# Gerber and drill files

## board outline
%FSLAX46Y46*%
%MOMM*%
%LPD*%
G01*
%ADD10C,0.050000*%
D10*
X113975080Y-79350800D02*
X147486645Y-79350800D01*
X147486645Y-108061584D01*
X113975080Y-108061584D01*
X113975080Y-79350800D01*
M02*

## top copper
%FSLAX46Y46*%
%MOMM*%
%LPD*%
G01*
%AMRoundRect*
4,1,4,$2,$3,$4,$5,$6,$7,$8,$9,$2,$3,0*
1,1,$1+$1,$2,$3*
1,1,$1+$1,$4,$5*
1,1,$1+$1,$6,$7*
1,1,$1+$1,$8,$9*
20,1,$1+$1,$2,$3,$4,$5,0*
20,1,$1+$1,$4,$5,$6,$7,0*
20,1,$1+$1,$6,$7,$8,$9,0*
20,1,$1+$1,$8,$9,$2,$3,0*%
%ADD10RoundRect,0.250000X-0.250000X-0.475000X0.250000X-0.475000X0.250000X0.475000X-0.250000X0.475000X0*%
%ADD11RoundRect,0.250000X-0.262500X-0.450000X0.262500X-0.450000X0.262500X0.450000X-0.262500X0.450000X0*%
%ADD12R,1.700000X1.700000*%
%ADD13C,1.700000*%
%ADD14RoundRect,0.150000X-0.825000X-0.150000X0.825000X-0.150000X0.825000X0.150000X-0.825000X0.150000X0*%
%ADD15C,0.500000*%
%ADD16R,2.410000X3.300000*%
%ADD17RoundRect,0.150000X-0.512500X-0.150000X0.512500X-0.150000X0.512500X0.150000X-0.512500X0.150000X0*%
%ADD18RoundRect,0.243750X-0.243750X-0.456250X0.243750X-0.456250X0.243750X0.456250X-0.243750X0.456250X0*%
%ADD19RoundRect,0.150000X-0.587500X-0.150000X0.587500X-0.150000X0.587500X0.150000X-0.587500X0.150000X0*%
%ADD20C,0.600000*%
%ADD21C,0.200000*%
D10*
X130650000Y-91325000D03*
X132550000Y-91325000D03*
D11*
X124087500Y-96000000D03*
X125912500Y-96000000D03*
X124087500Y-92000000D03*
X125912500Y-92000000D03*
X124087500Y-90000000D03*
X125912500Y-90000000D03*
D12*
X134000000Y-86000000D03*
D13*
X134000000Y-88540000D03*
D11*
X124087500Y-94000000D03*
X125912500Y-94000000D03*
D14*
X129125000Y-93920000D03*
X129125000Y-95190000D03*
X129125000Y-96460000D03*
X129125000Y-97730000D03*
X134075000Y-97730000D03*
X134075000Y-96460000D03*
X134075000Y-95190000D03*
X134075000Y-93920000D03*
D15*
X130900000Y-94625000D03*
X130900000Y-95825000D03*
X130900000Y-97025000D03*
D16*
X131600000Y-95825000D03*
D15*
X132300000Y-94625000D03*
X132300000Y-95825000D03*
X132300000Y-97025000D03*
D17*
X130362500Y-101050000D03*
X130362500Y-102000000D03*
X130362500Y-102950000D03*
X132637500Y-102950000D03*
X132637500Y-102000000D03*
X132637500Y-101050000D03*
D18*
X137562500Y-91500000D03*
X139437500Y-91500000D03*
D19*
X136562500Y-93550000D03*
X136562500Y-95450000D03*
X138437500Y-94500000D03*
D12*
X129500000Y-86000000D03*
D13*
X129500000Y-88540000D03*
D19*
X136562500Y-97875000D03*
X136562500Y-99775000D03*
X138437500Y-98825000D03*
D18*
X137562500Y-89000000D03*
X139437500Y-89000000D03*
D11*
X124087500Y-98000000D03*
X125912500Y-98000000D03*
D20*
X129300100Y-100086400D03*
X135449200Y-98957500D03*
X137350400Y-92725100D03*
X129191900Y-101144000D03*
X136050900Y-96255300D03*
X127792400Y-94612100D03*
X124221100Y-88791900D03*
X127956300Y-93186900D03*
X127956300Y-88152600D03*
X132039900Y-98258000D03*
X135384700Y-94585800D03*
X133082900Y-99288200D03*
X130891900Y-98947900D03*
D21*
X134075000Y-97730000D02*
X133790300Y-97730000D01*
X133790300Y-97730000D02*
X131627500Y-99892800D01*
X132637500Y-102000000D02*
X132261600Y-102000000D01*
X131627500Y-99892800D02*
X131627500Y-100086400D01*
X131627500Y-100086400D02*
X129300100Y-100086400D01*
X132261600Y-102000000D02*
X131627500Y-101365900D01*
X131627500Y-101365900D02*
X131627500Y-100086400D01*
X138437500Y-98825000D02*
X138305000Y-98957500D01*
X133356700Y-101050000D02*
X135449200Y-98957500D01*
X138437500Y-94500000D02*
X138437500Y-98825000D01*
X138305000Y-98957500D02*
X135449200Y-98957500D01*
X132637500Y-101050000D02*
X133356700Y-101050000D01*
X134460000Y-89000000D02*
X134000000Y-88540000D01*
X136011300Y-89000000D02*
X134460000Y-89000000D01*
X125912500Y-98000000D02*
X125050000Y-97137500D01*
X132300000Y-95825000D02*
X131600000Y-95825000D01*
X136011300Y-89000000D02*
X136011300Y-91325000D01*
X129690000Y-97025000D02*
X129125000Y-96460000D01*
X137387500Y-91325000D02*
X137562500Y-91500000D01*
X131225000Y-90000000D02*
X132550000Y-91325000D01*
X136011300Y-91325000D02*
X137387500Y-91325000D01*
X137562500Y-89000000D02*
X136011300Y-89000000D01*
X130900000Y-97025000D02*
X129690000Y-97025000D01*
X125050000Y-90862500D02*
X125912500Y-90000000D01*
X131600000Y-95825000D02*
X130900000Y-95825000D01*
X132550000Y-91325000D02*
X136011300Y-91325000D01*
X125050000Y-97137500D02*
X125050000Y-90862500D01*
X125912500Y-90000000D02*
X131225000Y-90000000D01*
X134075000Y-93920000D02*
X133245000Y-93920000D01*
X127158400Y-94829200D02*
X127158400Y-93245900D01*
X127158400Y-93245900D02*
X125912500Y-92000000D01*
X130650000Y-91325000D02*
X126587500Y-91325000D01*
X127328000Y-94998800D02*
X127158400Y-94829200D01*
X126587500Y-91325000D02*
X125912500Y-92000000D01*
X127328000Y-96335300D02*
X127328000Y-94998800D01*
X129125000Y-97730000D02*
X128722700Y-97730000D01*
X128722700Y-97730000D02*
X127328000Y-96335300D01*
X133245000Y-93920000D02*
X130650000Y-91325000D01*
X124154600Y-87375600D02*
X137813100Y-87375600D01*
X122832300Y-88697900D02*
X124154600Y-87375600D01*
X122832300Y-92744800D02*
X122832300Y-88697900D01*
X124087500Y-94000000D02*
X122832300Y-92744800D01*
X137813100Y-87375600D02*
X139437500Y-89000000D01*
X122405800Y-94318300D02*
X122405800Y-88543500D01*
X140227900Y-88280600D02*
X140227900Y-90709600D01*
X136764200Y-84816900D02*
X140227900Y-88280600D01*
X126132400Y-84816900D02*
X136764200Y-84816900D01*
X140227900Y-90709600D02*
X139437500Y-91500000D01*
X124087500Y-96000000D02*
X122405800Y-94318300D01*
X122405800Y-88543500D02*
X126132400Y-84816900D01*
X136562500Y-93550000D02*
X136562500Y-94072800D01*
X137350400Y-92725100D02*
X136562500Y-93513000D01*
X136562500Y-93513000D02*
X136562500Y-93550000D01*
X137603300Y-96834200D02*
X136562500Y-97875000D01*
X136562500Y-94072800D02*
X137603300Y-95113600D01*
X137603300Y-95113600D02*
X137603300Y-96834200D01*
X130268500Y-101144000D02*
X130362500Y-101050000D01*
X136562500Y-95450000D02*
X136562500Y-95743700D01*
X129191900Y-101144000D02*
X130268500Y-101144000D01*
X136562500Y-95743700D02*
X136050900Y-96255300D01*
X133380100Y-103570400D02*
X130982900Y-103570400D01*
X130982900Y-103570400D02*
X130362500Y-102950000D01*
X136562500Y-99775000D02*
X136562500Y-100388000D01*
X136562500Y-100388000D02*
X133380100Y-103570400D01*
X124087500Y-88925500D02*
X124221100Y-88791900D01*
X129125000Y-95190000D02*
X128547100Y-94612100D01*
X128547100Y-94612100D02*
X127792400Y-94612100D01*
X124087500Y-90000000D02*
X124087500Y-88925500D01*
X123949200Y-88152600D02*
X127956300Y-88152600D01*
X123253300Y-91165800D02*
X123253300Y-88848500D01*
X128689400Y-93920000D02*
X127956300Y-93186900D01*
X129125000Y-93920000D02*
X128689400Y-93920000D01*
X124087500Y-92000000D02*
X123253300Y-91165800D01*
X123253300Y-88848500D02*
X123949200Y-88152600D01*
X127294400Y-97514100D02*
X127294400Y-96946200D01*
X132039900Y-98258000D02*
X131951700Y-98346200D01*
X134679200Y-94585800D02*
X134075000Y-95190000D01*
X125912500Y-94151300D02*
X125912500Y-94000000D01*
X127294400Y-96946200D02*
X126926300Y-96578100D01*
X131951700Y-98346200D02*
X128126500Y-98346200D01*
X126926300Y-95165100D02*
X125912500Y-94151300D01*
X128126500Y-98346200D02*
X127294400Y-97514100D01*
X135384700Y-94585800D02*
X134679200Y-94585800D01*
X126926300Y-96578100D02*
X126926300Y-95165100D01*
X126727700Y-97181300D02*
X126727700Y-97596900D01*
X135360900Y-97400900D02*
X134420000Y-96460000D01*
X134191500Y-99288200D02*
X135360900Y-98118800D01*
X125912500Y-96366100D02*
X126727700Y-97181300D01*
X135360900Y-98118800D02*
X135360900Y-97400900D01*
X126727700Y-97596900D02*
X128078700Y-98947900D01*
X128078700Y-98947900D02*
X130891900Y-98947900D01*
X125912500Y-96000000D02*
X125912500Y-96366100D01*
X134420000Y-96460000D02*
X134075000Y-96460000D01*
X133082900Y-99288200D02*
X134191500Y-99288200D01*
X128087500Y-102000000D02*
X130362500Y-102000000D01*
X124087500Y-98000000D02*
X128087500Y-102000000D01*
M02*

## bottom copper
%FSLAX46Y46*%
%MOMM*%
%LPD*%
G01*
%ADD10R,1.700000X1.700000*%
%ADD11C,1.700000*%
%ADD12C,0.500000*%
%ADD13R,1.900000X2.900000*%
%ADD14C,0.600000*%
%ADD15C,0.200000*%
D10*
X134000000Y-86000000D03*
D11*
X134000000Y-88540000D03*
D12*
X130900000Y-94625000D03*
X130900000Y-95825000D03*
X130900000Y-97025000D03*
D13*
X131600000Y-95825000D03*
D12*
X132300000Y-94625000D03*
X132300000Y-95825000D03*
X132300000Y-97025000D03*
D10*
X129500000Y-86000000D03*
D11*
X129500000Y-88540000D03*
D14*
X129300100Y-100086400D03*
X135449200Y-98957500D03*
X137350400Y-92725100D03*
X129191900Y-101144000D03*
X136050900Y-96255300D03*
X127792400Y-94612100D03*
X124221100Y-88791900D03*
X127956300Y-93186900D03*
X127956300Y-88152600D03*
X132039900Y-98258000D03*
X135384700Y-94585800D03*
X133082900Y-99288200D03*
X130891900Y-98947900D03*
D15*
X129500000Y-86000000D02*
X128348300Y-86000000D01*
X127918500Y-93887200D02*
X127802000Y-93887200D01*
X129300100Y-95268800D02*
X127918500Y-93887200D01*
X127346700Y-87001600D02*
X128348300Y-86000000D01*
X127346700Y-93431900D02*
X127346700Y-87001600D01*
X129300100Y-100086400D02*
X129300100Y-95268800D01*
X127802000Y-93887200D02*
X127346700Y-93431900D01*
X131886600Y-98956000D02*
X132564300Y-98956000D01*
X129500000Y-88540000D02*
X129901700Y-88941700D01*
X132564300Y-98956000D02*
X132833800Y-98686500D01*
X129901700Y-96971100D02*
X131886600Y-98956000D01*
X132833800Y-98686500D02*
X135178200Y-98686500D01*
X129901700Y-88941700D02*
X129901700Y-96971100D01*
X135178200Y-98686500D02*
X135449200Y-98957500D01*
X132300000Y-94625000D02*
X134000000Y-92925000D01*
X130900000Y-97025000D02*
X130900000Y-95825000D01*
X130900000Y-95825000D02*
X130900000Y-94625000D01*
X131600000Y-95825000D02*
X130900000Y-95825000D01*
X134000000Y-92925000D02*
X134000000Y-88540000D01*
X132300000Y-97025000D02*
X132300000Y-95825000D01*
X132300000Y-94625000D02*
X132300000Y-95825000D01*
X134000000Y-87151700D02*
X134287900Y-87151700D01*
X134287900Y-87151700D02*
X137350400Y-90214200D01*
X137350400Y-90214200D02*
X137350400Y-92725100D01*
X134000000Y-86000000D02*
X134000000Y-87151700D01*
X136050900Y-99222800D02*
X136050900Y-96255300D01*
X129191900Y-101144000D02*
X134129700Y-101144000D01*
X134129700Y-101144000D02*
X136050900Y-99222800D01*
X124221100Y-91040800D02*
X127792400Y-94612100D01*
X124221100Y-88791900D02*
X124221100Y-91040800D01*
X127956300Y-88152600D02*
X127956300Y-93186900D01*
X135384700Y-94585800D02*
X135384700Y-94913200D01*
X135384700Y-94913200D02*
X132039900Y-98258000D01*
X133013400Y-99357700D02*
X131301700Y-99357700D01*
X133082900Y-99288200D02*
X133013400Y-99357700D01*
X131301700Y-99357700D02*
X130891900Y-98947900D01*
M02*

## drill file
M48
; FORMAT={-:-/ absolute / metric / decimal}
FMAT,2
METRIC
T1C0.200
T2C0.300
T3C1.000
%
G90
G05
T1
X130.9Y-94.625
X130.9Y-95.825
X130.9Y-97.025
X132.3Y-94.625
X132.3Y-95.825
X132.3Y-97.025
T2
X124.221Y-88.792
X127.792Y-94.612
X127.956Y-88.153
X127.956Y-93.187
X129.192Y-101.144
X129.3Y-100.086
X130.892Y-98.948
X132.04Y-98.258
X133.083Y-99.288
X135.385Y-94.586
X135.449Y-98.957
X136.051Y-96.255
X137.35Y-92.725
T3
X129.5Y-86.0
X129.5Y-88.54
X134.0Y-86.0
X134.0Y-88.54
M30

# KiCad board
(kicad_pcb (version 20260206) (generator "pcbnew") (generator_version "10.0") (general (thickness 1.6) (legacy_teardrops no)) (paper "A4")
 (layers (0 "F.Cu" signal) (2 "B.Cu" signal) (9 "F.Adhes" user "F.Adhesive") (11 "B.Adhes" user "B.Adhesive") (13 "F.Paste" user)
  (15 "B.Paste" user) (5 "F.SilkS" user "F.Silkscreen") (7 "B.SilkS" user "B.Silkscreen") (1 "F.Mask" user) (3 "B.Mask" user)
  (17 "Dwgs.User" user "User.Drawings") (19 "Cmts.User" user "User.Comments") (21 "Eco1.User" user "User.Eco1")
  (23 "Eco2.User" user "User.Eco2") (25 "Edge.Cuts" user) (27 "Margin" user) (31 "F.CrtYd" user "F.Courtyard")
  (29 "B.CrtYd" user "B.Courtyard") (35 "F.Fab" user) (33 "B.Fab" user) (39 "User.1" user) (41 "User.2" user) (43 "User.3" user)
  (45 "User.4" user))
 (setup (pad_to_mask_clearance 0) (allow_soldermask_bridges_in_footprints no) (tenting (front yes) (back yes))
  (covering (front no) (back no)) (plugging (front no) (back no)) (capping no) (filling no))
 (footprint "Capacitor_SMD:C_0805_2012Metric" (layer "F.Cu") (at 131.6 91.325)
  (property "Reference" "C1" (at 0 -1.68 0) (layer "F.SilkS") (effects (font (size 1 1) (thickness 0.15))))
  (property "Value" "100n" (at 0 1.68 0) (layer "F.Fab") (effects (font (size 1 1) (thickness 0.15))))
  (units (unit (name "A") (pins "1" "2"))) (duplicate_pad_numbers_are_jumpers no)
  (pad "1" smd roundrect (at -0.95 0) (size 1 1.45) (layers "F.Cu" "F.Mask" "F.Paste") (roundrect_rratio 0.25) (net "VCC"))
  (pad "2" smd roundrect (at 0.95 0) (size 1 1.45) (layers "F.Cu" "F.Mask" "F.Paste") (roundrect_rratio 0.25) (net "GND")))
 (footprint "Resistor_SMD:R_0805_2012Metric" (layer "F.Cu") (at 125 96)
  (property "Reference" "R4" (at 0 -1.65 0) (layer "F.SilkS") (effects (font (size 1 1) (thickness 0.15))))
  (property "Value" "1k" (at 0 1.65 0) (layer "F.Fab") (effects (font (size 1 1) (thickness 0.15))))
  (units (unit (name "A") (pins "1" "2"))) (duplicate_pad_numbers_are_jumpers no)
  (pad "1" smd roundrect (at -0.9125 0) (size 1.025 1.4) (layers "F.Cu" "F.Mask" "F.Paste") (roundrect_rratio 0.243902) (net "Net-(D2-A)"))
  (pad "2" smd roundrect (at 0.9125 0) (size 1.025 1.4) (layers "F.Cu" "F.Mask" "F.Paste") (roundrect_rratio 0.243902)
   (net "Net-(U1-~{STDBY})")))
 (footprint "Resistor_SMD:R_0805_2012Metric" (layer "F.Cu") (at 125 92)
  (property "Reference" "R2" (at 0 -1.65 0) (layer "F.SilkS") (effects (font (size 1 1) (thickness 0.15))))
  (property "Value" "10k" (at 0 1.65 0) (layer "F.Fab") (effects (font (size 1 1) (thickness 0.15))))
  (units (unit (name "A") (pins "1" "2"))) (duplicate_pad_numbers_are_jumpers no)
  (pad "1" smd roundrect (at -0.9125 0) (size 1.025 1.4) (layers "F.Cu" "F.Mask" "F.Paste") (roundrect_rratio 0.243902)
   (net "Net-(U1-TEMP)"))
  (pad "2" smd roundrect (at 0.9125 0) (size 1.025 1.4) (layers "F.Cu" "F.Mask" "F.Paste") (roundrect_rratio 0.243902) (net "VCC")))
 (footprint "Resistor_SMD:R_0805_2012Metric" (layer "F.Cu") (at 125 90)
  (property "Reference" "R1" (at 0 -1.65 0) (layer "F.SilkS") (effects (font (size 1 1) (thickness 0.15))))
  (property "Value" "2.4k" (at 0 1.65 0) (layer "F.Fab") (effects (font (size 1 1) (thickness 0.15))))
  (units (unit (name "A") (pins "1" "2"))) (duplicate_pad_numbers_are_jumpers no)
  (pad "1" smd roundrect (at -0.9125 0) (size 1.025 1.4) (layers "F.Cu" "F.Mask" "F.Paste") (roundrect_rratio 0.243902)
   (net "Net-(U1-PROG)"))
  (pad "2" smd roundrect (at 0.9125 0) (size 1.025 1.4) (layers "F.Cu" "F.Mask" "F.Paste") (roundrect_rratio 0.243902) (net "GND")))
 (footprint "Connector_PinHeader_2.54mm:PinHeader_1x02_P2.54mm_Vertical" (layer "F.Cu") (at 134 86)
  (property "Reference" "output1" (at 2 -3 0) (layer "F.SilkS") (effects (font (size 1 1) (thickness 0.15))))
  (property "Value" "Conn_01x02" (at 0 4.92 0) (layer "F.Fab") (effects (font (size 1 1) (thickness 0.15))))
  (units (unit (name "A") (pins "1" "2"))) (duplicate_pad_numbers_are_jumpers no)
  (pad "1" thru_hole rect (at 0 0) (size 1.7 1.7) (drill 1) (layers "*.Cu" "*.Mask") (remove_unused_layers no) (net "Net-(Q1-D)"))
  (pad "2" thru_hole circle (at 0 2.54) (size 1.7 1.7) (drill 1) (layers "*.Cu" "*.Mask") (remove_unused_layers no) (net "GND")))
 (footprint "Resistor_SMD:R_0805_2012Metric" (layer "F.Cu") (at 125 94)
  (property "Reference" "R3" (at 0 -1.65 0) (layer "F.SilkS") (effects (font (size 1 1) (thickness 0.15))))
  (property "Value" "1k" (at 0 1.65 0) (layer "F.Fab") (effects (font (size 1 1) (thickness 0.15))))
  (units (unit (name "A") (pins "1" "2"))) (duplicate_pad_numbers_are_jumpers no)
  (pad "1" smd roundrect (at -0.9125 0) (size 1.025 1.4) (layers "F.Cu" "F.Mask" "F.Paste") (roundrect_rratio 0.243902) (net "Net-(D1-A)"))
  (pad "2" smd roundrect (at 0.9125 0) (size 1.025 1.4) (layers "F.Cu" "F.Mask" "F.Paste") (roundrect_rratio 0.243902)
   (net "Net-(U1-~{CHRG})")))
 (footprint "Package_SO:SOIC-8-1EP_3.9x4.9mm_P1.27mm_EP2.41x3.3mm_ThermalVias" (layer "F.Cu") (at 131.6 95.825)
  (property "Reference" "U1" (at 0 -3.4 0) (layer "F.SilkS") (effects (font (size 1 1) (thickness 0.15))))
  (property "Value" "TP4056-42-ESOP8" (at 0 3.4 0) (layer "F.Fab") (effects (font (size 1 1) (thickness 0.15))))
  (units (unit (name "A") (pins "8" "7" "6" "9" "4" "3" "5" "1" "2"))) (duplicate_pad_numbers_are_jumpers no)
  (pad "" smd roundrect (at -0.6 -0.825) (size 1.01 1.38) (layers "F.Paste") (roundrect_rratio 0.247525))
  (pad "" smd roundrect (at -0.6 0.825) (size 1.01 1.38) (layers "F.Paste") (roundrect_rratio 0.247525))
  (pad "" smd roundrect (at 0.6 -0.825) (size 1.01 1.38) (layers "F.Paste") (roundrect_rratio 0.247525))
  (pad "" smd roundrect (at 0.6 0.825) (size 1.01 1.38) (layers "F.Paste") (roundrect_rratio 0.247525))
  (pad "1" smd roundrect (at -2.475 -1.905) (size 1.95 0.6) (layers "F.Cu" "F.Mask" "F.Paste") (roundrect_rratio 0.25) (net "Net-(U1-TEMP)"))
  (pad "2" smd roundrect (at -2.475 -0.635) (size 1.95 0.6) (layers "F.Cu" "F.Mask" "F.Paste") (roundrect_rratio 0.25) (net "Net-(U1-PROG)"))
  (pad "3" smd roundrect (at -2.475 0.635) (size 1.95 0.6) (layers "F.Cu" "F.Mask" "F.Paste") (roundrect_rratio 0.25) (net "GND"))
  (pad "4" smd roundrect (at -2.475 1.905) (size 1.95 0.6) (layers "F.Cu" "F.Mask" "F.Paste") (roundrect_rratio 0.25) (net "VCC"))
  (pad "5" smd roundrect (at 2.475 1.905) (size 1.95 0.6) (layers "F.Cu" "F.Mask" "F.Paste") (roundrect_rratio 0.25) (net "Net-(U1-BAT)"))
  (pad "6" smd roundrect (at 2.475 0.635) (size 1.95 0.6) (layers "F.Cu" "F.Mask" "F.Paste") (roundrect_rratio 0.25)
   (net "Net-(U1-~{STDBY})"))
  (pad "7" smd roundrect (at 2.475 -0.635) (size 1.95 0.6) (layers "F.Cu" "F.Mask" "F.Paste") (roundrect_rratio 0.25)
   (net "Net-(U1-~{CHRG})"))
  (pad "8" smd roundrect (at 2.475 -1.905) (size 1.95 0.6) (layers "F.Cu" "F.Mask" "F.Paste") (roundrect_rratio 0.25) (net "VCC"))
  (pad "9" thru_hole circle (at -0.7 -1.2) (size 0.5 0.5) (drill 0.2) (layers "*.Cu") (remove_unused_layers no) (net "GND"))
  (pad "9" thru_hole circle (at -0.7 0) (size 0.5 0.5) (drill 0.2) (layers "*.Cu") (remove_unused_layers no) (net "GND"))
  (pad "9" thru_hole circle (at -0.7 1.2) (size 0.5 0.5) (drill 0.2) (layers "*.Cu") (remove_unused_layers no) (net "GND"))
  (pad "9" smd rect (at 0 0) (size 1.9 2.9) (layers "B.Cu") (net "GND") (zone_connect 2))
  (pad "9" smd rect (at 0 0) (size 2.41 3.3) (layers "F.Cu" "F.Mask") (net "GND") (zone_connect 2))
  (pad "9" thru_hole circle (at 0.7 -1.2) (size 0.5 0.5) (drill 0.2) (layers "*.Cu") (remove_unused_layers no) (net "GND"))
  (pad "9" thru_hole circle (at 0.7 0) (size 0.5 0.5) (drill 0.2) (layers "*.Cu") (remove_unused_layers no) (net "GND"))
  (pad "9" thru_hole circle (at 0.7 1.2) (size 0.5 0.5) (drill 0.2) (layers "*.Cu") (remove_unused_layers no) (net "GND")))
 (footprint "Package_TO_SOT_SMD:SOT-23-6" (layer "F.Cu") (at 131.5 102)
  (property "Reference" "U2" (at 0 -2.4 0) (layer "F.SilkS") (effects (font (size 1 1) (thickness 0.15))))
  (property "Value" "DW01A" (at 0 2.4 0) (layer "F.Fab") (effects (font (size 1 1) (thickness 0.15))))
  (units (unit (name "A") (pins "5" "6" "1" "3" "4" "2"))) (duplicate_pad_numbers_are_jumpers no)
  (pad "1" smd roundrect (at -1.1375 -0.95) (size 1.325 0.6) (layers "F.Cu" "F.Mask" "F.Paste") (roundrect_rratio 0.25) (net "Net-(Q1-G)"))
  (pad "2" smd roundrect (at -1.1375 0) (size 1.325 0.6) (layers "F.Cu" "F.Mask" "F.Paste") (roundrect_rratio 0.25) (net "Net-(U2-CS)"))
  (pad "3" smd roundrect (at -1.1375 0.95) (size 1.325 0.6) (layers "F.Cu" "F.Mask" "F.Paste") (roundrect_rratio 0.25) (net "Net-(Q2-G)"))
  (pad "4" smd roundrect (at 1.1375 0.95) (size 1.325 0.6) (layers "F.Cu" "F.Mask" "F.Paste") (roundrect_rratio 0.25)
   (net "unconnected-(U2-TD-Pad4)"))
  (pad "5" smd roundrect (at 1.1375 0) (size 1.325 0.6) (layers "F.Cu" "F.Mask" "F.Paste") (roundrect_rratio 0.25) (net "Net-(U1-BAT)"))
  (pad "6" smd roundrect (at 1.1375 -0.95) (size 1.325 0.6) (layers "F.Cu" "F.Mask" "F.Paste") (roundrect_rratio 0.25) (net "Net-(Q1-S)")))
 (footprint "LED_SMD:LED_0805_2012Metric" (layer "F.Cu") (at 138.5 91.5)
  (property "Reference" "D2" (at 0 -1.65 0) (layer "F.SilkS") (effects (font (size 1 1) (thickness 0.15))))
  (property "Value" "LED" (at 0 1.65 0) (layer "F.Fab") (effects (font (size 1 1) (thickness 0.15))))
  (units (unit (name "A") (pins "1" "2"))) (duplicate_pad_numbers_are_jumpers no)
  (pad "1" smd roundrect (at -0.9375 0) (size 0.975 1.4) (layers "F.Cu" "F.Mask" "F.Paste") (roundrect_rratio 0.25) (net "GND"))
  (pad "2" smd roundrect (at 0.9375 0) (size 0.975 1.4) (layers "F.Cu" "F.Mask" "F.Paste") (roundrect_rratio 0.25) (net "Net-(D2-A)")))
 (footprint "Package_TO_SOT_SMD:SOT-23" (layer "F.Cu") (at 137.5 94.5)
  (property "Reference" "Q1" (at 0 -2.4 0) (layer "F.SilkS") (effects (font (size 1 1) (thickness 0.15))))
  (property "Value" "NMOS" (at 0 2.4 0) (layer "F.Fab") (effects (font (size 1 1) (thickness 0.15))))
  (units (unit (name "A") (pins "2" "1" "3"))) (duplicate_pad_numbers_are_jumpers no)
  (pad "1" smd roundrect (at -0.9375 -0.95) (size 1.475 0.6) (layers "F.Cu" "F.Mask" "F.Paste") (roundrect_rratio 0.25) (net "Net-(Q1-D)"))
  (pad "2" smd roundrect (at -0.9375 0.95) (size 1.475 0.6) (layers "F.Cu" "F.Mask" "F.Paste") (roundrect_rratio 0.25) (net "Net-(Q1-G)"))
  (pad "3" smd roundrect (at 0.9375 0) (size 1.475 0.6) (layers "F.Cu" "F.Mask" "F.Paste") (roundrect_rratio 0.25) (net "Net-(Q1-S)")))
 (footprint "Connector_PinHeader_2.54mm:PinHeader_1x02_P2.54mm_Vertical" (layer "F.Cu") (at 129.5 86)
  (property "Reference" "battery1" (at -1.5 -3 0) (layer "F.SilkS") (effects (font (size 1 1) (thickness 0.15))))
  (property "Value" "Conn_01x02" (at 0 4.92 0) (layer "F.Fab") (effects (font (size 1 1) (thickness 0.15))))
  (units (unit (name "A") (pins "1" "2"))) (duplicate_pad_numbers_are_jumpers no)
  (pad "1" thru_hole rect (at 0 0) (size 1.7 1.7) (drill 1) (layers "*.Cu" "*.Mask") (remove_unused_layers no) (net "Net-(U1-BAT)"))
  (pad "2" thru_hole circle (at 0 2.54) (size 1.7 1.7) (drill 1) (layers "*.Cu" "*.Mask") (remove_unused_layers no) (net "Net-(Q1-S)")))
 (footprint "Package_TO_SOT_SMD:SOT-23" (layer "F.Cu") (at 137.5 98.825)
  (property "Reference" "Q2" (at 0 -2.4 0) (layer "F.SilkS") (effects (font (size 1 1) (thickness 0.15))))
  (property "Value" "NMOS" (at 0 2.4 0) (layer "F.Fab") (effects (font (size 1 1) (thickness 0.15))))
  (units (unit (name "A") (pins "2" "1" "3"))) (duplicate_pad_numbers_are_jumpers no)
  (pad "1" smd roundrect (at -0.9375 -0.95) (size 1.475 0.6) (layers "F.Cu" "F.Mask" "F.Paste") (roundrect_rratio 0.25) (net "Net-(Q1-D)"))
  (pad "2" smd roundrect (at -0.9375 0.95) (size 1.475 0.6) (layers "F.Cu" "F.Mask" "F.Paste") (roundrect_rratio 0.25) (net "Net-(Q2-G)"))
  (pad "3" smd roundrect (at 0.9375 0) (size 1.475 0.6) (layers "F.Cu" "F.Mask" "F.Paste") (roundrect_rratio 0.25) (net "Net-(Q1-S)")))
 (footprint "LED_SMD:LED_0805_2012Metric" (layer "F.Cu") (at 138.5 89)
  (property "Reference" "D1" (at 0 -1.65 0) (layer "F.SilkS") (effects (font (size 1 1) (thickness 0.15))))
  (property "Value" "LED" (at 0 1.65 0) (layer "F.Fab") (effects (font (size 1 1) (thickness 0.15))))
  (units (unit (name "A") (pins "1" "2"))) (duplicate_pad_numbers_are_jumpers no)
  (pad "1" smd roundrect (at -0.9375 0) (size 0.975 1.4) (layers "F.Cu" "F.Mask" "F.Paste") (roundrect_rratio 0.25) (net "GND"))
  (pad "2" smd roundrect (at 0.9375 0) (size 0.975 1.4) (layers "F.Cu" "F.Mask" "F.Paste") (roundrect_rratio 0.25) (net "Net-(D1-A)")))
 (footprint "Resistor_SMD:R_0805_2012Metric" (layer "F.Cu") (at 125 98)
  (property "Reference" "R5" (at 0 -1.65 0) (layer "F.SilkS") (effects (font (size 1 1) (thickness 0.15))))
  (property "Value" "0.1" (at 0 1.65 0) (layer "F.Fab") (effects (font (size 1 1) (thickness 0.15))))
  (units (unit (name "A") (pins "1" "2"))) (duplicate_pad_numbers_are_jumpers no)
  (pad "1" smd roundrect (at -0.9125 0) (size 1.025 1.4) (layers "F.Cu" "F.Mask" "F.Paste") (roundrect_rratio 0.243902) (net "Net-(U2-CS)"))
  (pad "2" smd roundrect (at 0.9125 0) (size 1.025 1.4) (layers "F.Cu" "F.Mask" "F.Paste") (roundrect_rratio 0.243902) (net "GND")))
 (gr_rect (start 113.97508 79.3508) (end 147.486645 108.061584) (stroke (width 0.05) (type default)) (fill no) (layer "Edge.Cuts"))
 (segment (start 134.075 97.73) (end 133.7903 97.73) (width 0.2) (layer "F.Cu") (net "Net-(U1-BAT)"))
 (segment (start 133.7903 97.73) (end 131.6275 99.8928) (width 0.2) (layer "F.Cu") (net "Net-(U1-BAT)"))
 (segment (start 132.6375 102) (end 132.2616 102) (width 0.2) (layer "F.Cu") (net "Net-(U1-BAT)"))
 (segment (start 131.6275 99.8928) (end 131.6275 100.0864) (width 0.2) (layer "F.Cu") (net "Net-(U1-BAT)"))
 (segment (start 131.6275 100.0864) (end 129.3001 100.0864) (width 0.2) (layer "F.Cu") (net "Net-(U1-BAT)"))
 (segment (start 132.2616 102) (end 131.6275 101.3659) (width 0.2) (layer "F.Cu") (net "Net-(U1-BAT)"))
 (segment (start 131.6275 101.3659) (end 131.6275 100.0864) (width 0.2) (layer "F.Cu") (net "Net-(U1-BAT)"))
 (via (at 129.3001 100.0864) (size 0.6) (drill 0.3) (layers "F.Cu" "B.Cu") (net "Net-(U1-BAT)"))
 (segment (start 129.5 86) (end 128.3483 86) (width 0.2) (layer "B.Cu") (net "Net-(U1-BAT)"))
 (segment (start 127.9185 93.8872) (end 127.802 93.8872) (width 0.2) (layer "B.Cu") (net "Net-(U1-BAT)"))
 (segment (start 129.3001 95.2688) (end 127.9185 93.8872) (width 0.2) (layer "B.Cu") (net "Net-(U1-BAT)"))
 (segment (start 127.3467 87.0016) (end 128.3483 86) (width 0.2) (layer "B.Cu") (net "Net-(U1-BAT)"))
 (segment (start 127.3467 93.4319) (end 127.3467 87.0016) (width 0.2) (layer "B.Cu") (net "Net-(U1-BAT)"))
 (segment (start 129.3001 100.0864) (end 129.3001 95.2688) (width 0.2) (layer "B.Cu") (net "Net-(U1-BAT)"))
 (segment (start 127.802 93.8872) (end 127.3467 93.4319) (width 0.2) (layer "B.Cu") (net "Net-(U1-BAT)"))
 (segment (start 138.4375 98.825) (end 138.305 98.9575) (width 0.2) (layer "F.Cu") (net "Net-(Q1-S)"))
 (segment (start 133.3567 101.05) (end 135.4492 98.9575) (width 0.2) (layer "F.Cu") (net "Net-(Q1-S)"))
 (segment (start 138.4375 94.5) (end 138.4375 98.825) (width 0.2) (layer "F.Cu") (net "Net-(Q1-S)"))
 (segment (start 138.305 98.9575) (end 135.4492 98.9575) (width 0.2) (layer "F.Cu") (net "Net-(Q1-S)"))
 (segment (start 132.6375 101.05) (end 133.3567 101.05) (width 0.2) (layer "F.Cu") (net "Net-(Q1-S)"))
 (via (at 135.4492 98.9575) (size 0.6) (drill 0.3) (layers "F.Cu" "B.Cu") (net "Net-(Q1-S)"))
 (segment (start 131.8866 98.956) (end 132.5643 98.956) (width 0.2) (layer "B.Cu") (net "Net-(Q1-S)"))
 (segment (start 129.5 88.54) (end 129.9017 88.9417) (width 0.2) (layer "B.Cu") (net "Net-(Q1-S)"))
 (segment (start 132.5643 98.956) (end 132.8338 98.6865) (width 0.2) (layer "B.Cu") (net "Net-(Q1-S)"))
 (segment (start 129.9017 96.9711) (end 131.8866 98.956) (width 0.2) (layer "B.Cu") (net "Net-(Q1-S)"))
 (segment (start 132.8338 98.6865) (end 135.1782 98.6865) (width 0.2) (layer "B.Cu") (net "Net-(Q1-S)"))
 (segment (start 129.9017 88.9417) (end 129.9017 96.9711) (width 0.2) (layer "B.Cu") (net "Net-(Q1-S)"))
 (segment (start 135.1782 98.6865) (end 135.4492 98.9575) (width 0.2) (layer "B.Cu") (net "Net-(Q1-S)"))
 (segment (start 134.46 89) (end 134 88.54) (width 0.2) (layer "F.Cu") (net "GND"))
 (segment (start 136.0113 89) (end 134.46 89) (width 0.2) (layer "F.Cu") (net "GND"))
 (segment (start 125.9125 98) (end 125.05 97.1375) (width 0.2) (layer "F.Cu") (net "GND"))
 (segment (start 132.3 95.825) (end 131.6 95.825) (width 0.2) (layer "F.Cu") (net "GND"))
 (segment (start 136.0113 89) (end 136.0113 91.325) (width 0.2) (layer "F.Cu") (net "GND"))
 (segment (start 129.69 97.025) (end 129.125 96.46) (width 0.2) (layer "F.Cu") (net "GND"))
 (segment (start 137.3875 91.325) (end 137.5625 91.5) (width 0.2) (layer "F.Cu") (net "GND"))
 (segment (start 131.225 90) (end 132.55 91.325) (width 0.2) (layer "F.Cu") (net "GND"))
 (segment (start 136.0113 91.325) (end 137.3875 91.325) (width 0.2) (layer "F.Cu") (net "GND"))
 (segment (start 137.5625 89) (end 136.0113 89) (width 0.2) (layer "F.Cu") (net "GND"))
 (segment (start 130.9 97.025) (end 129.69 97.025) (width 0.2) (layer "F.Cu") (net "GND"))
 (segment (start 125.05 90.8625) (end 125.9125 90) (width 0.2) (layer "F.Cu") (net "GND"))
 (segment (start 131.6 95.825) (end 130.9 95.825) (width 0.2) (layer "F.Cu") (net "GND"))
 (segment (start 132.55 91.325) (end 136.0113 91.325) (width 0.2) (layer "F.Cu") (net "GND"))
 (segment (start 125.05 97.1375) (end 125.05 90.8625) (width 0.2) (layer "F.Cu") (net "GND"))
 (segment (start 125.9125 90) (end 131.225 90) (width 0.2) (layer "F.Cu") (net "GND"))
 (segment (start 132.3 94.625) (end 134 92.925) (width 0.2) (layer "B.Cu") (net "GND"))
 (segment (start 130.9 97.025) (end 130.9 95.825) (width 0.2) (layer "B.Cu") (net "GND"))
 (segment (start 130.9 95.825) (end 130.9 94.625) (width 0.2) (layer "B.Cu") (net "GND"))
 (segment (start 131.6 95.825) (end 130.9 95.825) (width 0.2) (layer "B.Cu") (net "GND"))
 (segment (start 134 92.925) (end 134 88.54) (width 0.2) (layer "B.Cu") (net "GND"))
 (segment (start 132.3 97.025) (end 132.3 95.825) (width 0.2) (layer "B.Cu") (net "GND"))
 (segment (start 132.3 94.625) (end 132.3 95.825) (width 0.2) (layer "B.Cu") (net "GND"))
 (segment (start 134.075 93.92) (end 133.245 93.92) (width 0.2) (layer "F.Cu") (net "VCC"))
 (segment (start 127.1584 94.8292) (end 127.1584 93.2459) (width 0.2) (layer "F.Cu") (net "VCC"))
 (segment (start 127.1584 93.2459) (end 125.9125 92) (width 0.2) (layer "F.Cu") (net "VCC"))
 (segment (start 130.65 91.325) (end 126.5875 91.325) (width 0.2) (layer "F.Cu") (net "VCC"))
 (segment (start 127.328 94.9988) (end 127.1584 94.8292) (width 0.2) (layer "F.Cu") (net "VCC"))
 (segment (start 126.5875 91.325) (end 125.9125 92) (width 0.2) (layer "F.Cu") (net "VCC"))
 (segment (start 127.328 96.3353) (end 127.328 94.9988) (width 0.2) (layer "F.Cu") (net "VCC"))
 (segment (start 129.125 97.73) (end 128.7227 97.73) (width 0.2) (layer "F.Cu") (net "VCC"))
 (segment (start 128.7227 97.73) (end 127.328 96.3353) (width 0.2) (layer "F.Cu") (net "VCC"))
 (segment (start 133.245 93.92) (end 130.65 91.325) (width 0.2) (layer "F.Cu") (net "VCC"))
 (segment (start 124.1546 87.3756) (end 137.8131 87.3756) (width 0.2) (layer "F.Cu") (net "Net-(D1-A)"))
 (segment (start 122.8323 88.6979) (end 124.1546 87.3756) (width 0.2) (layer "F.Cu") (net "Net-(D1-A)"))
 (segment (start 122.8323 92.7448) (end 122.8323 88.6979) (width 0.2) (layer "F.Cu") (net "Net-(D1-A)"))
 (segment (start 124.0875 94) (end 122.8323 92.7448) (width 0.2) (layer "F.Cu") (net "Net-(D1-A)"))
 (segment (start 137.8131 87.3756) (end 139.4375 89) (width 0.2) (layer "F.Cu") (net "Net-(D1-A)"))
 (segment (start 122.4058 94.3183) (end 122.4058 88.5435) (width 0.2) (layer "F.Cu") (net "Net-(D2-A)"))
 (segment (start 140.2279 88.2806) (end 140.2279 90.7096) (width 0.2) (layer "F.Cu") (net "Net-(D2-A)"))
 (segment (start 136.7642 84.8169) (end 140.2279 88.2806) (width 0.2) (layer "F.Cu") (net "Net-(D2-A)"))
 (segment (start 126.1324 84.8169) (end 136.7642 84.8169) (width 0.2) (layer "F.Cu") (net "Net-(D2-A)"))
 (segment (start 140.2279 90.7096) (end 139.4375 91.5) (width 0.2) (layer "F.Cu") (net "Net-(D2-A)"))
 (segment (start 124.0875 96) (end 122.4058 94.3183) (width 0.2) (layer "F.Cu") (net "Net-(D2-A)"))
 (segment (start 122.4058 88.5435) (end 126.1324 84.8169) (width 0.2) (layer "F.Cu") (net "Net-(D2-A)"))
 (segment (start 136.5625 93.55) (end 136.5625 94.0728) (width 0.2) (layer "F.Cu") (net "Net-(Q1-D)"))
 (segment (start 137.3504 92.7251) (end 136.5625 93.513) (width 0.2) (layer "F.Cu") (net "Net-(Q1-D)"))
 (segment (start 136.5625 93.513) (end 136.5625 93.55) (width 0.2) (layer "F.Cu") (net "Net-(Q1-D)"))
 (segment (start 137.6033 96.8342) (end 136.5625 97.875) (width 0.2) (layer "F.Cu") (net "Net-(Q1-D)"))
 (segment (start 136.5625 94.0728) (end 137.6033 95.1136) (width 0.2) (layer "F.Cu") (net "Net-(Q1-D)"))
 (segment (start 137.6033 95.1136) (end 137.6033 96.8342) (width 0.2) (layer "F.Cu") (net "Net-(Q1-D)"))
 (via (at 137.3504 92.7251) (size 0.6) (drill 0.3) (layers "F.Cu" "B.Cu") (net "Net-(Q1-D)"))
 (segment (start 134 87.1517) (end 134.2879 87.1517) (width 0.2) (layer "B.Cu") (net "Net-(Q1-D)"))
 (segment (start 134.2879 87.1517) (end 137.3504 90.2142) (width 0.2) (layer "B.Cu") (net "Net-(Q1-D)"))
 (segment (start 137.3504 90.2142) (end 137.3504 92.7251) (width 0.2) (layer "B.Cu") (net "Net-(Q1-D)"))
 (segment (start 134 86) (end 134 87.1517) (width 0.2) (layer "B.Cu") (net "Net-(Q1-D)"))
 (segment (start 130.2685 101.144) (end 130.3625 101.05) (width 0.2) (layer "F.Cu") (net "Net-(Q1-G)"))
 (segment (start 136.5625 95.45) (end 136.5625 95.7437) (width 0.2) (layer "F.Cu") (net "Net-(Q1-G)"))
 (segment (start 129.1919 101.144) (end 130.2685 101.144) (width 0.2) (layer "F.Cu") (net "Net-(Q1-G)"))
 (segment (start 136.5625 95.7437) (end 136.0509 96.2553) (width 0.2) (layer "F.Cu") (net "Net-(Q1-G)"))
 (via (at 129.1919 101.144) (size 0.6) (drill 0.3) (layers "F.Cu" "B.Cu") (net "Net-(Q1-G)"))
 (via (at 136.0509 96.2553) (size 0.6) (drill 0.3) (layers "F.Cu" "B.Cu") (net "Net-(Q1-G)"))
 (segment (start 136.0509 99.2228) (end 136.0509 96.2553) (width 0.2) (layer "B.Cu") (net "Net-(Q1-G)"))
 (segment (start 129.1919 101.144) (end 134.1297 101.144) (width 0.2) (layer "B.Cu") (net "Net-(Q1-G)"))
 (segment (start 134.1297 101.144) (end 136.0509 99.2228) (width 0.2) (layer "B.Cu") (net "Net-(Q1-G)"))
 (segment (start 133.3801 103.5704) (end 130.9829 103.5704) (width 0.2) (layer "F.Cu") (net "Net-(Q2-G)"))
 (segment (start 130.9829 103.5704) (end 130.3625 102.95) (width 0.2) (layer "F.Cu") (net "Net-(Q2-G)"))
 (segment (start 136.5625 99.775) (end 136.5625 100.388) (width 0.2) (layer "F.Cu") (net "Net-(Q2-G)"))
 (segment (start 136.5625 100.388) (end 133.3801 103.5704) (width 0.2) (layer "F.Cu") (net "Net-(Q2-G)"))
 (segment (start 124.0875 88.9255) (end 124.2211 88.7919) (width 0.2) (layer "F.Cu") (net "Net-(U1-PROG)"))
 (segment (start 129.125 95.19) (end 128.5471 94.6121) (width 0.2) (layer "F.Cu") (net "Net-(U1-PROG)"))
 (segment (start 128.5471 94.6121) (end 127.7924 94.6121) (width 0.2) (layer "F.Cu") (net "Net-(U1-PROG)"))
 (segment (start 124.0875 90) (end 124.0875 88.9255) (width 0.2) (layer "F.Cu") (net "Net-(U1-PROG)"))
 (via (at 127.7924 94.6121) (size 0.6) (drill 0.3) (layers "F.Cu" "B.Cu") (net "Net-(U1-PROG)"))
 (via (at 124.2211 88.7919) (size 0.6) (drill 0.3) (layers "F.Cu" "B.Cu") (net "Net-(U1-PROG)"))
 (segment (start 124.2211 91.0408) (end 127.7924 94.6121) (width 0.2) (layer "B.Cu") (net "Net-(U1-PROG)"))
 (segment (start 124.2211 88.7919) (end 124.2211 91.0408) (width 0.2) (layer "B.Cu") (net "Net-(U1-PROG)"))
 (segment (start 123.9492 88.1526) (end 127.9563 88.1526) (width 0.2) (layer "F.Cu") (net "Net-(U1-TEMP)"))
 (segment (start 123.2533 91.1658) (end 123.2533 88.8485) (width 0.2) (layer "F.Cu") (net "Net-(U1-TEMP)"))
 (segment (start 128.6894 93.92) (end 127.9563 93.1869) (width 0.2) (layer "F.Cu") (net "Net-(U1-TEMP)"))
 (segment (start 129.125 93.92) (end 128.6894 93.92) (width 0.2) (layer "F.Cu") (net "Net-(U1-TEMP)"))
 (segment (start 124.0875 92) (end 123.2533 91.1658) (width 0.2) (layer "F.Cu") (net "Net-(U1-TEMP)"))
 (segment (start 123.2533 88.8485) (end 123.9492 88.1526) (width 0.2) (layer "F.Cu") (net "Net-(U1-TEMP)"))
 (via (at 127.9563 93.1869) (size 0.6) (drill 0.3) (layers "F.Cu" "B.Cu") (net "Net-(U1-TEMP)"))
 (via (at 127.9563 88.1526) (size 0.6) (drill 0.3) (layers "F.Cu" "B.Cu") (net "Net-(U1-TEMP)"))
 (segment (start 127.9563 88.1526) (end 127.9563 93.1869) (width 0.2) (layer "B.Cu") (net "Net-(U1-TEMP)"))
 (segment (start 127.2944 97.5141) (end 127.2944 96.9462) (width 0.2) (layer "F.Cu") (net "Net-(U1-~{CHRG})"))
 (segment (start 132.0399 98.258) (end 131.9517 98.3462) (width 0.2) (layer "F.Cu") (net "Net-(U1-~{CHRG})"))
 (segment (start 134.6792 94.5858) (end 134.075 95.19) (width 0.2) (layer "F.Cu") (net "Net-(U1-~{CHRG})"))
 (segment (start 125.9125 94.1513) (end 125.9125 94) (width 0.2) (layer "F.Cu") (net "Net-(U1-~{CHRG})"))
 (segment (start 127.2944 96.9462) (end 126.9263 96.5781) (width 0.2) (layer "F.Cu") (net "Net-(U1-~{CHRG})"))
 (segment (start 131.9517 98.3462) (end 128.1265 98.3462) (width 0.2) (layer "F.Cu") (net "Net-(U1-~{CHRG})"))
 (segment (start 126.9263 95.1651) (end 125.9125 94.1513) (width 0.2) (layer "F.Cu") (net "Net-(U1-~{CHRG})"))
 (segment (start 128.1265 98.3462) (end 127.2944 97.5141) (width 0.2) (layer "F.Cu") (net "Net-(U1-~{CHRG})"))
 (segment (start 135.3847 94.5858) (end 134.6792 94.5858) (width 0.2) (layer "F.Cu") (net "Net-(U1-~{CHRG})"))
 (segment (start 126.9263 96.5781) (end 126.9263 95.1651) (width 0.2) (layer "F.Cu") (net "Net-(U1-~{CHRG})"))
 (via (at 132.0399 98.258) (size 0.6) (drill 0.3) (layers "F.Cu" "B.Cu") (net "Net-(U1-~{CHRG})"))
 (via (at 135.3847 94.5858) (size 0.6) (drill 0.3) (layers "F.Cu" "B.Cu") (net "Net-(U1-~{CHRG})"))
 (segment (start 135.3847 94.5858) (end 135.3847 94.9132) (width 0.2) (layer "B.Cu") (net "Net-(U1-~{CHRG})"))
 (segment (start 135.3847 94.9132) (end 132.0399 98.258) (width 0.2) (layer "B.Cu") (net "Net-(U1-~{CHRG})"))
 (segment (start 126.7277 97.1813) (end 126.7277 97.5969) (width 0.2) (layer "F.Cu") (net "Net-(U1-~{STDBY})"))
 (segment (start 135.3609 97.4009) (end 134.42 96.46) (width 0.2) (layer "F.Cu") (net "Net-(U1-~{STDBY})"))
 (segment (start 134.1915 99.2882) (end 135.3609 98.1188) (width 0.2) (layer "F.Cu") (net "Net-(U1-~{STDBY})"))
 (segment (start 125.9125 96.3661) (end 126.7277 97.1813) (width 0.2) (layer "F.Cu") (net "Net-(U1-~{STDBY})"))
 (segment (start 135.3609 98.1188) (end 135.3609 97.4009) (width 0.2) (layer "F.Cu") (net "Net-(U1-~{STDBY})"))
 (segment (start 126.7277 97.5969) (end 128.0787 98.9479) (width 0.2) (layer "F.Cu") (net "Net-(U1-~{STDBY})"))
 (segment (start 128.0787 98.9479) (end 130.8919 98.9479) (width 0.2) (layer "F.Cu") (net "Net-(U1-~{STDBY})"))
 (segment (start 125.9125 96) (end 125.9125 96.3661) (width 0.2) (layer "F.Cu") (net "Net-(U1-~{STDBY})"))
 (segment (start 134.42 96.46) (end 134.075 96.46) (width 0.2) (layer "F.Cu") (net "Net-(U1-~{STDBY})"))
 (segment (start 133.0829 99.2882) (end 134.1915 99.2882) (width 0.2) (layer "F.Cu") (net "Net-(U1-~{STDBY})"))
 (via (at 133.0829 99.2882) (size 0.6) (drill 0.3) (layers "F.Cu" "B.Cu") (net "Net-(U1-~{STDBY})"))
 (via (at 130.8919 98.9479) (size 0.6) (drill 0.3) (layers "F.Cu" "B.Cu") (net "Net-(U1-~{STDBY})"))
 (segment (start 133.0134 99.3577) (end 131.3017 99.3577) (width 0.2) (layer "B.Cu") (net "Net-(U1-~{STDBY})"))
 (segment (start 133.0829 99.2882) (end 133.0134 99.3577) (width 0.2) (layer "B.Cu") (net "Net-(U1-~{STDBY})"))
 (segment (start 131.3017 99.3577) (end 130.8919 98.9479) (width 0.2) (layer "B.Cu") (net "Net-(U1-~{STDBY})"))
 (segment (start 128.0875 102) (end 130.3625 102) (width 0.2) (layer "F.Cu") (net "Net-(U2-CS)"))
 (segment (start 124.0875 98) (end 128.0875 102) (width 0.2) (layer "F.Cu") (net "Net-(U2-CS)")))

